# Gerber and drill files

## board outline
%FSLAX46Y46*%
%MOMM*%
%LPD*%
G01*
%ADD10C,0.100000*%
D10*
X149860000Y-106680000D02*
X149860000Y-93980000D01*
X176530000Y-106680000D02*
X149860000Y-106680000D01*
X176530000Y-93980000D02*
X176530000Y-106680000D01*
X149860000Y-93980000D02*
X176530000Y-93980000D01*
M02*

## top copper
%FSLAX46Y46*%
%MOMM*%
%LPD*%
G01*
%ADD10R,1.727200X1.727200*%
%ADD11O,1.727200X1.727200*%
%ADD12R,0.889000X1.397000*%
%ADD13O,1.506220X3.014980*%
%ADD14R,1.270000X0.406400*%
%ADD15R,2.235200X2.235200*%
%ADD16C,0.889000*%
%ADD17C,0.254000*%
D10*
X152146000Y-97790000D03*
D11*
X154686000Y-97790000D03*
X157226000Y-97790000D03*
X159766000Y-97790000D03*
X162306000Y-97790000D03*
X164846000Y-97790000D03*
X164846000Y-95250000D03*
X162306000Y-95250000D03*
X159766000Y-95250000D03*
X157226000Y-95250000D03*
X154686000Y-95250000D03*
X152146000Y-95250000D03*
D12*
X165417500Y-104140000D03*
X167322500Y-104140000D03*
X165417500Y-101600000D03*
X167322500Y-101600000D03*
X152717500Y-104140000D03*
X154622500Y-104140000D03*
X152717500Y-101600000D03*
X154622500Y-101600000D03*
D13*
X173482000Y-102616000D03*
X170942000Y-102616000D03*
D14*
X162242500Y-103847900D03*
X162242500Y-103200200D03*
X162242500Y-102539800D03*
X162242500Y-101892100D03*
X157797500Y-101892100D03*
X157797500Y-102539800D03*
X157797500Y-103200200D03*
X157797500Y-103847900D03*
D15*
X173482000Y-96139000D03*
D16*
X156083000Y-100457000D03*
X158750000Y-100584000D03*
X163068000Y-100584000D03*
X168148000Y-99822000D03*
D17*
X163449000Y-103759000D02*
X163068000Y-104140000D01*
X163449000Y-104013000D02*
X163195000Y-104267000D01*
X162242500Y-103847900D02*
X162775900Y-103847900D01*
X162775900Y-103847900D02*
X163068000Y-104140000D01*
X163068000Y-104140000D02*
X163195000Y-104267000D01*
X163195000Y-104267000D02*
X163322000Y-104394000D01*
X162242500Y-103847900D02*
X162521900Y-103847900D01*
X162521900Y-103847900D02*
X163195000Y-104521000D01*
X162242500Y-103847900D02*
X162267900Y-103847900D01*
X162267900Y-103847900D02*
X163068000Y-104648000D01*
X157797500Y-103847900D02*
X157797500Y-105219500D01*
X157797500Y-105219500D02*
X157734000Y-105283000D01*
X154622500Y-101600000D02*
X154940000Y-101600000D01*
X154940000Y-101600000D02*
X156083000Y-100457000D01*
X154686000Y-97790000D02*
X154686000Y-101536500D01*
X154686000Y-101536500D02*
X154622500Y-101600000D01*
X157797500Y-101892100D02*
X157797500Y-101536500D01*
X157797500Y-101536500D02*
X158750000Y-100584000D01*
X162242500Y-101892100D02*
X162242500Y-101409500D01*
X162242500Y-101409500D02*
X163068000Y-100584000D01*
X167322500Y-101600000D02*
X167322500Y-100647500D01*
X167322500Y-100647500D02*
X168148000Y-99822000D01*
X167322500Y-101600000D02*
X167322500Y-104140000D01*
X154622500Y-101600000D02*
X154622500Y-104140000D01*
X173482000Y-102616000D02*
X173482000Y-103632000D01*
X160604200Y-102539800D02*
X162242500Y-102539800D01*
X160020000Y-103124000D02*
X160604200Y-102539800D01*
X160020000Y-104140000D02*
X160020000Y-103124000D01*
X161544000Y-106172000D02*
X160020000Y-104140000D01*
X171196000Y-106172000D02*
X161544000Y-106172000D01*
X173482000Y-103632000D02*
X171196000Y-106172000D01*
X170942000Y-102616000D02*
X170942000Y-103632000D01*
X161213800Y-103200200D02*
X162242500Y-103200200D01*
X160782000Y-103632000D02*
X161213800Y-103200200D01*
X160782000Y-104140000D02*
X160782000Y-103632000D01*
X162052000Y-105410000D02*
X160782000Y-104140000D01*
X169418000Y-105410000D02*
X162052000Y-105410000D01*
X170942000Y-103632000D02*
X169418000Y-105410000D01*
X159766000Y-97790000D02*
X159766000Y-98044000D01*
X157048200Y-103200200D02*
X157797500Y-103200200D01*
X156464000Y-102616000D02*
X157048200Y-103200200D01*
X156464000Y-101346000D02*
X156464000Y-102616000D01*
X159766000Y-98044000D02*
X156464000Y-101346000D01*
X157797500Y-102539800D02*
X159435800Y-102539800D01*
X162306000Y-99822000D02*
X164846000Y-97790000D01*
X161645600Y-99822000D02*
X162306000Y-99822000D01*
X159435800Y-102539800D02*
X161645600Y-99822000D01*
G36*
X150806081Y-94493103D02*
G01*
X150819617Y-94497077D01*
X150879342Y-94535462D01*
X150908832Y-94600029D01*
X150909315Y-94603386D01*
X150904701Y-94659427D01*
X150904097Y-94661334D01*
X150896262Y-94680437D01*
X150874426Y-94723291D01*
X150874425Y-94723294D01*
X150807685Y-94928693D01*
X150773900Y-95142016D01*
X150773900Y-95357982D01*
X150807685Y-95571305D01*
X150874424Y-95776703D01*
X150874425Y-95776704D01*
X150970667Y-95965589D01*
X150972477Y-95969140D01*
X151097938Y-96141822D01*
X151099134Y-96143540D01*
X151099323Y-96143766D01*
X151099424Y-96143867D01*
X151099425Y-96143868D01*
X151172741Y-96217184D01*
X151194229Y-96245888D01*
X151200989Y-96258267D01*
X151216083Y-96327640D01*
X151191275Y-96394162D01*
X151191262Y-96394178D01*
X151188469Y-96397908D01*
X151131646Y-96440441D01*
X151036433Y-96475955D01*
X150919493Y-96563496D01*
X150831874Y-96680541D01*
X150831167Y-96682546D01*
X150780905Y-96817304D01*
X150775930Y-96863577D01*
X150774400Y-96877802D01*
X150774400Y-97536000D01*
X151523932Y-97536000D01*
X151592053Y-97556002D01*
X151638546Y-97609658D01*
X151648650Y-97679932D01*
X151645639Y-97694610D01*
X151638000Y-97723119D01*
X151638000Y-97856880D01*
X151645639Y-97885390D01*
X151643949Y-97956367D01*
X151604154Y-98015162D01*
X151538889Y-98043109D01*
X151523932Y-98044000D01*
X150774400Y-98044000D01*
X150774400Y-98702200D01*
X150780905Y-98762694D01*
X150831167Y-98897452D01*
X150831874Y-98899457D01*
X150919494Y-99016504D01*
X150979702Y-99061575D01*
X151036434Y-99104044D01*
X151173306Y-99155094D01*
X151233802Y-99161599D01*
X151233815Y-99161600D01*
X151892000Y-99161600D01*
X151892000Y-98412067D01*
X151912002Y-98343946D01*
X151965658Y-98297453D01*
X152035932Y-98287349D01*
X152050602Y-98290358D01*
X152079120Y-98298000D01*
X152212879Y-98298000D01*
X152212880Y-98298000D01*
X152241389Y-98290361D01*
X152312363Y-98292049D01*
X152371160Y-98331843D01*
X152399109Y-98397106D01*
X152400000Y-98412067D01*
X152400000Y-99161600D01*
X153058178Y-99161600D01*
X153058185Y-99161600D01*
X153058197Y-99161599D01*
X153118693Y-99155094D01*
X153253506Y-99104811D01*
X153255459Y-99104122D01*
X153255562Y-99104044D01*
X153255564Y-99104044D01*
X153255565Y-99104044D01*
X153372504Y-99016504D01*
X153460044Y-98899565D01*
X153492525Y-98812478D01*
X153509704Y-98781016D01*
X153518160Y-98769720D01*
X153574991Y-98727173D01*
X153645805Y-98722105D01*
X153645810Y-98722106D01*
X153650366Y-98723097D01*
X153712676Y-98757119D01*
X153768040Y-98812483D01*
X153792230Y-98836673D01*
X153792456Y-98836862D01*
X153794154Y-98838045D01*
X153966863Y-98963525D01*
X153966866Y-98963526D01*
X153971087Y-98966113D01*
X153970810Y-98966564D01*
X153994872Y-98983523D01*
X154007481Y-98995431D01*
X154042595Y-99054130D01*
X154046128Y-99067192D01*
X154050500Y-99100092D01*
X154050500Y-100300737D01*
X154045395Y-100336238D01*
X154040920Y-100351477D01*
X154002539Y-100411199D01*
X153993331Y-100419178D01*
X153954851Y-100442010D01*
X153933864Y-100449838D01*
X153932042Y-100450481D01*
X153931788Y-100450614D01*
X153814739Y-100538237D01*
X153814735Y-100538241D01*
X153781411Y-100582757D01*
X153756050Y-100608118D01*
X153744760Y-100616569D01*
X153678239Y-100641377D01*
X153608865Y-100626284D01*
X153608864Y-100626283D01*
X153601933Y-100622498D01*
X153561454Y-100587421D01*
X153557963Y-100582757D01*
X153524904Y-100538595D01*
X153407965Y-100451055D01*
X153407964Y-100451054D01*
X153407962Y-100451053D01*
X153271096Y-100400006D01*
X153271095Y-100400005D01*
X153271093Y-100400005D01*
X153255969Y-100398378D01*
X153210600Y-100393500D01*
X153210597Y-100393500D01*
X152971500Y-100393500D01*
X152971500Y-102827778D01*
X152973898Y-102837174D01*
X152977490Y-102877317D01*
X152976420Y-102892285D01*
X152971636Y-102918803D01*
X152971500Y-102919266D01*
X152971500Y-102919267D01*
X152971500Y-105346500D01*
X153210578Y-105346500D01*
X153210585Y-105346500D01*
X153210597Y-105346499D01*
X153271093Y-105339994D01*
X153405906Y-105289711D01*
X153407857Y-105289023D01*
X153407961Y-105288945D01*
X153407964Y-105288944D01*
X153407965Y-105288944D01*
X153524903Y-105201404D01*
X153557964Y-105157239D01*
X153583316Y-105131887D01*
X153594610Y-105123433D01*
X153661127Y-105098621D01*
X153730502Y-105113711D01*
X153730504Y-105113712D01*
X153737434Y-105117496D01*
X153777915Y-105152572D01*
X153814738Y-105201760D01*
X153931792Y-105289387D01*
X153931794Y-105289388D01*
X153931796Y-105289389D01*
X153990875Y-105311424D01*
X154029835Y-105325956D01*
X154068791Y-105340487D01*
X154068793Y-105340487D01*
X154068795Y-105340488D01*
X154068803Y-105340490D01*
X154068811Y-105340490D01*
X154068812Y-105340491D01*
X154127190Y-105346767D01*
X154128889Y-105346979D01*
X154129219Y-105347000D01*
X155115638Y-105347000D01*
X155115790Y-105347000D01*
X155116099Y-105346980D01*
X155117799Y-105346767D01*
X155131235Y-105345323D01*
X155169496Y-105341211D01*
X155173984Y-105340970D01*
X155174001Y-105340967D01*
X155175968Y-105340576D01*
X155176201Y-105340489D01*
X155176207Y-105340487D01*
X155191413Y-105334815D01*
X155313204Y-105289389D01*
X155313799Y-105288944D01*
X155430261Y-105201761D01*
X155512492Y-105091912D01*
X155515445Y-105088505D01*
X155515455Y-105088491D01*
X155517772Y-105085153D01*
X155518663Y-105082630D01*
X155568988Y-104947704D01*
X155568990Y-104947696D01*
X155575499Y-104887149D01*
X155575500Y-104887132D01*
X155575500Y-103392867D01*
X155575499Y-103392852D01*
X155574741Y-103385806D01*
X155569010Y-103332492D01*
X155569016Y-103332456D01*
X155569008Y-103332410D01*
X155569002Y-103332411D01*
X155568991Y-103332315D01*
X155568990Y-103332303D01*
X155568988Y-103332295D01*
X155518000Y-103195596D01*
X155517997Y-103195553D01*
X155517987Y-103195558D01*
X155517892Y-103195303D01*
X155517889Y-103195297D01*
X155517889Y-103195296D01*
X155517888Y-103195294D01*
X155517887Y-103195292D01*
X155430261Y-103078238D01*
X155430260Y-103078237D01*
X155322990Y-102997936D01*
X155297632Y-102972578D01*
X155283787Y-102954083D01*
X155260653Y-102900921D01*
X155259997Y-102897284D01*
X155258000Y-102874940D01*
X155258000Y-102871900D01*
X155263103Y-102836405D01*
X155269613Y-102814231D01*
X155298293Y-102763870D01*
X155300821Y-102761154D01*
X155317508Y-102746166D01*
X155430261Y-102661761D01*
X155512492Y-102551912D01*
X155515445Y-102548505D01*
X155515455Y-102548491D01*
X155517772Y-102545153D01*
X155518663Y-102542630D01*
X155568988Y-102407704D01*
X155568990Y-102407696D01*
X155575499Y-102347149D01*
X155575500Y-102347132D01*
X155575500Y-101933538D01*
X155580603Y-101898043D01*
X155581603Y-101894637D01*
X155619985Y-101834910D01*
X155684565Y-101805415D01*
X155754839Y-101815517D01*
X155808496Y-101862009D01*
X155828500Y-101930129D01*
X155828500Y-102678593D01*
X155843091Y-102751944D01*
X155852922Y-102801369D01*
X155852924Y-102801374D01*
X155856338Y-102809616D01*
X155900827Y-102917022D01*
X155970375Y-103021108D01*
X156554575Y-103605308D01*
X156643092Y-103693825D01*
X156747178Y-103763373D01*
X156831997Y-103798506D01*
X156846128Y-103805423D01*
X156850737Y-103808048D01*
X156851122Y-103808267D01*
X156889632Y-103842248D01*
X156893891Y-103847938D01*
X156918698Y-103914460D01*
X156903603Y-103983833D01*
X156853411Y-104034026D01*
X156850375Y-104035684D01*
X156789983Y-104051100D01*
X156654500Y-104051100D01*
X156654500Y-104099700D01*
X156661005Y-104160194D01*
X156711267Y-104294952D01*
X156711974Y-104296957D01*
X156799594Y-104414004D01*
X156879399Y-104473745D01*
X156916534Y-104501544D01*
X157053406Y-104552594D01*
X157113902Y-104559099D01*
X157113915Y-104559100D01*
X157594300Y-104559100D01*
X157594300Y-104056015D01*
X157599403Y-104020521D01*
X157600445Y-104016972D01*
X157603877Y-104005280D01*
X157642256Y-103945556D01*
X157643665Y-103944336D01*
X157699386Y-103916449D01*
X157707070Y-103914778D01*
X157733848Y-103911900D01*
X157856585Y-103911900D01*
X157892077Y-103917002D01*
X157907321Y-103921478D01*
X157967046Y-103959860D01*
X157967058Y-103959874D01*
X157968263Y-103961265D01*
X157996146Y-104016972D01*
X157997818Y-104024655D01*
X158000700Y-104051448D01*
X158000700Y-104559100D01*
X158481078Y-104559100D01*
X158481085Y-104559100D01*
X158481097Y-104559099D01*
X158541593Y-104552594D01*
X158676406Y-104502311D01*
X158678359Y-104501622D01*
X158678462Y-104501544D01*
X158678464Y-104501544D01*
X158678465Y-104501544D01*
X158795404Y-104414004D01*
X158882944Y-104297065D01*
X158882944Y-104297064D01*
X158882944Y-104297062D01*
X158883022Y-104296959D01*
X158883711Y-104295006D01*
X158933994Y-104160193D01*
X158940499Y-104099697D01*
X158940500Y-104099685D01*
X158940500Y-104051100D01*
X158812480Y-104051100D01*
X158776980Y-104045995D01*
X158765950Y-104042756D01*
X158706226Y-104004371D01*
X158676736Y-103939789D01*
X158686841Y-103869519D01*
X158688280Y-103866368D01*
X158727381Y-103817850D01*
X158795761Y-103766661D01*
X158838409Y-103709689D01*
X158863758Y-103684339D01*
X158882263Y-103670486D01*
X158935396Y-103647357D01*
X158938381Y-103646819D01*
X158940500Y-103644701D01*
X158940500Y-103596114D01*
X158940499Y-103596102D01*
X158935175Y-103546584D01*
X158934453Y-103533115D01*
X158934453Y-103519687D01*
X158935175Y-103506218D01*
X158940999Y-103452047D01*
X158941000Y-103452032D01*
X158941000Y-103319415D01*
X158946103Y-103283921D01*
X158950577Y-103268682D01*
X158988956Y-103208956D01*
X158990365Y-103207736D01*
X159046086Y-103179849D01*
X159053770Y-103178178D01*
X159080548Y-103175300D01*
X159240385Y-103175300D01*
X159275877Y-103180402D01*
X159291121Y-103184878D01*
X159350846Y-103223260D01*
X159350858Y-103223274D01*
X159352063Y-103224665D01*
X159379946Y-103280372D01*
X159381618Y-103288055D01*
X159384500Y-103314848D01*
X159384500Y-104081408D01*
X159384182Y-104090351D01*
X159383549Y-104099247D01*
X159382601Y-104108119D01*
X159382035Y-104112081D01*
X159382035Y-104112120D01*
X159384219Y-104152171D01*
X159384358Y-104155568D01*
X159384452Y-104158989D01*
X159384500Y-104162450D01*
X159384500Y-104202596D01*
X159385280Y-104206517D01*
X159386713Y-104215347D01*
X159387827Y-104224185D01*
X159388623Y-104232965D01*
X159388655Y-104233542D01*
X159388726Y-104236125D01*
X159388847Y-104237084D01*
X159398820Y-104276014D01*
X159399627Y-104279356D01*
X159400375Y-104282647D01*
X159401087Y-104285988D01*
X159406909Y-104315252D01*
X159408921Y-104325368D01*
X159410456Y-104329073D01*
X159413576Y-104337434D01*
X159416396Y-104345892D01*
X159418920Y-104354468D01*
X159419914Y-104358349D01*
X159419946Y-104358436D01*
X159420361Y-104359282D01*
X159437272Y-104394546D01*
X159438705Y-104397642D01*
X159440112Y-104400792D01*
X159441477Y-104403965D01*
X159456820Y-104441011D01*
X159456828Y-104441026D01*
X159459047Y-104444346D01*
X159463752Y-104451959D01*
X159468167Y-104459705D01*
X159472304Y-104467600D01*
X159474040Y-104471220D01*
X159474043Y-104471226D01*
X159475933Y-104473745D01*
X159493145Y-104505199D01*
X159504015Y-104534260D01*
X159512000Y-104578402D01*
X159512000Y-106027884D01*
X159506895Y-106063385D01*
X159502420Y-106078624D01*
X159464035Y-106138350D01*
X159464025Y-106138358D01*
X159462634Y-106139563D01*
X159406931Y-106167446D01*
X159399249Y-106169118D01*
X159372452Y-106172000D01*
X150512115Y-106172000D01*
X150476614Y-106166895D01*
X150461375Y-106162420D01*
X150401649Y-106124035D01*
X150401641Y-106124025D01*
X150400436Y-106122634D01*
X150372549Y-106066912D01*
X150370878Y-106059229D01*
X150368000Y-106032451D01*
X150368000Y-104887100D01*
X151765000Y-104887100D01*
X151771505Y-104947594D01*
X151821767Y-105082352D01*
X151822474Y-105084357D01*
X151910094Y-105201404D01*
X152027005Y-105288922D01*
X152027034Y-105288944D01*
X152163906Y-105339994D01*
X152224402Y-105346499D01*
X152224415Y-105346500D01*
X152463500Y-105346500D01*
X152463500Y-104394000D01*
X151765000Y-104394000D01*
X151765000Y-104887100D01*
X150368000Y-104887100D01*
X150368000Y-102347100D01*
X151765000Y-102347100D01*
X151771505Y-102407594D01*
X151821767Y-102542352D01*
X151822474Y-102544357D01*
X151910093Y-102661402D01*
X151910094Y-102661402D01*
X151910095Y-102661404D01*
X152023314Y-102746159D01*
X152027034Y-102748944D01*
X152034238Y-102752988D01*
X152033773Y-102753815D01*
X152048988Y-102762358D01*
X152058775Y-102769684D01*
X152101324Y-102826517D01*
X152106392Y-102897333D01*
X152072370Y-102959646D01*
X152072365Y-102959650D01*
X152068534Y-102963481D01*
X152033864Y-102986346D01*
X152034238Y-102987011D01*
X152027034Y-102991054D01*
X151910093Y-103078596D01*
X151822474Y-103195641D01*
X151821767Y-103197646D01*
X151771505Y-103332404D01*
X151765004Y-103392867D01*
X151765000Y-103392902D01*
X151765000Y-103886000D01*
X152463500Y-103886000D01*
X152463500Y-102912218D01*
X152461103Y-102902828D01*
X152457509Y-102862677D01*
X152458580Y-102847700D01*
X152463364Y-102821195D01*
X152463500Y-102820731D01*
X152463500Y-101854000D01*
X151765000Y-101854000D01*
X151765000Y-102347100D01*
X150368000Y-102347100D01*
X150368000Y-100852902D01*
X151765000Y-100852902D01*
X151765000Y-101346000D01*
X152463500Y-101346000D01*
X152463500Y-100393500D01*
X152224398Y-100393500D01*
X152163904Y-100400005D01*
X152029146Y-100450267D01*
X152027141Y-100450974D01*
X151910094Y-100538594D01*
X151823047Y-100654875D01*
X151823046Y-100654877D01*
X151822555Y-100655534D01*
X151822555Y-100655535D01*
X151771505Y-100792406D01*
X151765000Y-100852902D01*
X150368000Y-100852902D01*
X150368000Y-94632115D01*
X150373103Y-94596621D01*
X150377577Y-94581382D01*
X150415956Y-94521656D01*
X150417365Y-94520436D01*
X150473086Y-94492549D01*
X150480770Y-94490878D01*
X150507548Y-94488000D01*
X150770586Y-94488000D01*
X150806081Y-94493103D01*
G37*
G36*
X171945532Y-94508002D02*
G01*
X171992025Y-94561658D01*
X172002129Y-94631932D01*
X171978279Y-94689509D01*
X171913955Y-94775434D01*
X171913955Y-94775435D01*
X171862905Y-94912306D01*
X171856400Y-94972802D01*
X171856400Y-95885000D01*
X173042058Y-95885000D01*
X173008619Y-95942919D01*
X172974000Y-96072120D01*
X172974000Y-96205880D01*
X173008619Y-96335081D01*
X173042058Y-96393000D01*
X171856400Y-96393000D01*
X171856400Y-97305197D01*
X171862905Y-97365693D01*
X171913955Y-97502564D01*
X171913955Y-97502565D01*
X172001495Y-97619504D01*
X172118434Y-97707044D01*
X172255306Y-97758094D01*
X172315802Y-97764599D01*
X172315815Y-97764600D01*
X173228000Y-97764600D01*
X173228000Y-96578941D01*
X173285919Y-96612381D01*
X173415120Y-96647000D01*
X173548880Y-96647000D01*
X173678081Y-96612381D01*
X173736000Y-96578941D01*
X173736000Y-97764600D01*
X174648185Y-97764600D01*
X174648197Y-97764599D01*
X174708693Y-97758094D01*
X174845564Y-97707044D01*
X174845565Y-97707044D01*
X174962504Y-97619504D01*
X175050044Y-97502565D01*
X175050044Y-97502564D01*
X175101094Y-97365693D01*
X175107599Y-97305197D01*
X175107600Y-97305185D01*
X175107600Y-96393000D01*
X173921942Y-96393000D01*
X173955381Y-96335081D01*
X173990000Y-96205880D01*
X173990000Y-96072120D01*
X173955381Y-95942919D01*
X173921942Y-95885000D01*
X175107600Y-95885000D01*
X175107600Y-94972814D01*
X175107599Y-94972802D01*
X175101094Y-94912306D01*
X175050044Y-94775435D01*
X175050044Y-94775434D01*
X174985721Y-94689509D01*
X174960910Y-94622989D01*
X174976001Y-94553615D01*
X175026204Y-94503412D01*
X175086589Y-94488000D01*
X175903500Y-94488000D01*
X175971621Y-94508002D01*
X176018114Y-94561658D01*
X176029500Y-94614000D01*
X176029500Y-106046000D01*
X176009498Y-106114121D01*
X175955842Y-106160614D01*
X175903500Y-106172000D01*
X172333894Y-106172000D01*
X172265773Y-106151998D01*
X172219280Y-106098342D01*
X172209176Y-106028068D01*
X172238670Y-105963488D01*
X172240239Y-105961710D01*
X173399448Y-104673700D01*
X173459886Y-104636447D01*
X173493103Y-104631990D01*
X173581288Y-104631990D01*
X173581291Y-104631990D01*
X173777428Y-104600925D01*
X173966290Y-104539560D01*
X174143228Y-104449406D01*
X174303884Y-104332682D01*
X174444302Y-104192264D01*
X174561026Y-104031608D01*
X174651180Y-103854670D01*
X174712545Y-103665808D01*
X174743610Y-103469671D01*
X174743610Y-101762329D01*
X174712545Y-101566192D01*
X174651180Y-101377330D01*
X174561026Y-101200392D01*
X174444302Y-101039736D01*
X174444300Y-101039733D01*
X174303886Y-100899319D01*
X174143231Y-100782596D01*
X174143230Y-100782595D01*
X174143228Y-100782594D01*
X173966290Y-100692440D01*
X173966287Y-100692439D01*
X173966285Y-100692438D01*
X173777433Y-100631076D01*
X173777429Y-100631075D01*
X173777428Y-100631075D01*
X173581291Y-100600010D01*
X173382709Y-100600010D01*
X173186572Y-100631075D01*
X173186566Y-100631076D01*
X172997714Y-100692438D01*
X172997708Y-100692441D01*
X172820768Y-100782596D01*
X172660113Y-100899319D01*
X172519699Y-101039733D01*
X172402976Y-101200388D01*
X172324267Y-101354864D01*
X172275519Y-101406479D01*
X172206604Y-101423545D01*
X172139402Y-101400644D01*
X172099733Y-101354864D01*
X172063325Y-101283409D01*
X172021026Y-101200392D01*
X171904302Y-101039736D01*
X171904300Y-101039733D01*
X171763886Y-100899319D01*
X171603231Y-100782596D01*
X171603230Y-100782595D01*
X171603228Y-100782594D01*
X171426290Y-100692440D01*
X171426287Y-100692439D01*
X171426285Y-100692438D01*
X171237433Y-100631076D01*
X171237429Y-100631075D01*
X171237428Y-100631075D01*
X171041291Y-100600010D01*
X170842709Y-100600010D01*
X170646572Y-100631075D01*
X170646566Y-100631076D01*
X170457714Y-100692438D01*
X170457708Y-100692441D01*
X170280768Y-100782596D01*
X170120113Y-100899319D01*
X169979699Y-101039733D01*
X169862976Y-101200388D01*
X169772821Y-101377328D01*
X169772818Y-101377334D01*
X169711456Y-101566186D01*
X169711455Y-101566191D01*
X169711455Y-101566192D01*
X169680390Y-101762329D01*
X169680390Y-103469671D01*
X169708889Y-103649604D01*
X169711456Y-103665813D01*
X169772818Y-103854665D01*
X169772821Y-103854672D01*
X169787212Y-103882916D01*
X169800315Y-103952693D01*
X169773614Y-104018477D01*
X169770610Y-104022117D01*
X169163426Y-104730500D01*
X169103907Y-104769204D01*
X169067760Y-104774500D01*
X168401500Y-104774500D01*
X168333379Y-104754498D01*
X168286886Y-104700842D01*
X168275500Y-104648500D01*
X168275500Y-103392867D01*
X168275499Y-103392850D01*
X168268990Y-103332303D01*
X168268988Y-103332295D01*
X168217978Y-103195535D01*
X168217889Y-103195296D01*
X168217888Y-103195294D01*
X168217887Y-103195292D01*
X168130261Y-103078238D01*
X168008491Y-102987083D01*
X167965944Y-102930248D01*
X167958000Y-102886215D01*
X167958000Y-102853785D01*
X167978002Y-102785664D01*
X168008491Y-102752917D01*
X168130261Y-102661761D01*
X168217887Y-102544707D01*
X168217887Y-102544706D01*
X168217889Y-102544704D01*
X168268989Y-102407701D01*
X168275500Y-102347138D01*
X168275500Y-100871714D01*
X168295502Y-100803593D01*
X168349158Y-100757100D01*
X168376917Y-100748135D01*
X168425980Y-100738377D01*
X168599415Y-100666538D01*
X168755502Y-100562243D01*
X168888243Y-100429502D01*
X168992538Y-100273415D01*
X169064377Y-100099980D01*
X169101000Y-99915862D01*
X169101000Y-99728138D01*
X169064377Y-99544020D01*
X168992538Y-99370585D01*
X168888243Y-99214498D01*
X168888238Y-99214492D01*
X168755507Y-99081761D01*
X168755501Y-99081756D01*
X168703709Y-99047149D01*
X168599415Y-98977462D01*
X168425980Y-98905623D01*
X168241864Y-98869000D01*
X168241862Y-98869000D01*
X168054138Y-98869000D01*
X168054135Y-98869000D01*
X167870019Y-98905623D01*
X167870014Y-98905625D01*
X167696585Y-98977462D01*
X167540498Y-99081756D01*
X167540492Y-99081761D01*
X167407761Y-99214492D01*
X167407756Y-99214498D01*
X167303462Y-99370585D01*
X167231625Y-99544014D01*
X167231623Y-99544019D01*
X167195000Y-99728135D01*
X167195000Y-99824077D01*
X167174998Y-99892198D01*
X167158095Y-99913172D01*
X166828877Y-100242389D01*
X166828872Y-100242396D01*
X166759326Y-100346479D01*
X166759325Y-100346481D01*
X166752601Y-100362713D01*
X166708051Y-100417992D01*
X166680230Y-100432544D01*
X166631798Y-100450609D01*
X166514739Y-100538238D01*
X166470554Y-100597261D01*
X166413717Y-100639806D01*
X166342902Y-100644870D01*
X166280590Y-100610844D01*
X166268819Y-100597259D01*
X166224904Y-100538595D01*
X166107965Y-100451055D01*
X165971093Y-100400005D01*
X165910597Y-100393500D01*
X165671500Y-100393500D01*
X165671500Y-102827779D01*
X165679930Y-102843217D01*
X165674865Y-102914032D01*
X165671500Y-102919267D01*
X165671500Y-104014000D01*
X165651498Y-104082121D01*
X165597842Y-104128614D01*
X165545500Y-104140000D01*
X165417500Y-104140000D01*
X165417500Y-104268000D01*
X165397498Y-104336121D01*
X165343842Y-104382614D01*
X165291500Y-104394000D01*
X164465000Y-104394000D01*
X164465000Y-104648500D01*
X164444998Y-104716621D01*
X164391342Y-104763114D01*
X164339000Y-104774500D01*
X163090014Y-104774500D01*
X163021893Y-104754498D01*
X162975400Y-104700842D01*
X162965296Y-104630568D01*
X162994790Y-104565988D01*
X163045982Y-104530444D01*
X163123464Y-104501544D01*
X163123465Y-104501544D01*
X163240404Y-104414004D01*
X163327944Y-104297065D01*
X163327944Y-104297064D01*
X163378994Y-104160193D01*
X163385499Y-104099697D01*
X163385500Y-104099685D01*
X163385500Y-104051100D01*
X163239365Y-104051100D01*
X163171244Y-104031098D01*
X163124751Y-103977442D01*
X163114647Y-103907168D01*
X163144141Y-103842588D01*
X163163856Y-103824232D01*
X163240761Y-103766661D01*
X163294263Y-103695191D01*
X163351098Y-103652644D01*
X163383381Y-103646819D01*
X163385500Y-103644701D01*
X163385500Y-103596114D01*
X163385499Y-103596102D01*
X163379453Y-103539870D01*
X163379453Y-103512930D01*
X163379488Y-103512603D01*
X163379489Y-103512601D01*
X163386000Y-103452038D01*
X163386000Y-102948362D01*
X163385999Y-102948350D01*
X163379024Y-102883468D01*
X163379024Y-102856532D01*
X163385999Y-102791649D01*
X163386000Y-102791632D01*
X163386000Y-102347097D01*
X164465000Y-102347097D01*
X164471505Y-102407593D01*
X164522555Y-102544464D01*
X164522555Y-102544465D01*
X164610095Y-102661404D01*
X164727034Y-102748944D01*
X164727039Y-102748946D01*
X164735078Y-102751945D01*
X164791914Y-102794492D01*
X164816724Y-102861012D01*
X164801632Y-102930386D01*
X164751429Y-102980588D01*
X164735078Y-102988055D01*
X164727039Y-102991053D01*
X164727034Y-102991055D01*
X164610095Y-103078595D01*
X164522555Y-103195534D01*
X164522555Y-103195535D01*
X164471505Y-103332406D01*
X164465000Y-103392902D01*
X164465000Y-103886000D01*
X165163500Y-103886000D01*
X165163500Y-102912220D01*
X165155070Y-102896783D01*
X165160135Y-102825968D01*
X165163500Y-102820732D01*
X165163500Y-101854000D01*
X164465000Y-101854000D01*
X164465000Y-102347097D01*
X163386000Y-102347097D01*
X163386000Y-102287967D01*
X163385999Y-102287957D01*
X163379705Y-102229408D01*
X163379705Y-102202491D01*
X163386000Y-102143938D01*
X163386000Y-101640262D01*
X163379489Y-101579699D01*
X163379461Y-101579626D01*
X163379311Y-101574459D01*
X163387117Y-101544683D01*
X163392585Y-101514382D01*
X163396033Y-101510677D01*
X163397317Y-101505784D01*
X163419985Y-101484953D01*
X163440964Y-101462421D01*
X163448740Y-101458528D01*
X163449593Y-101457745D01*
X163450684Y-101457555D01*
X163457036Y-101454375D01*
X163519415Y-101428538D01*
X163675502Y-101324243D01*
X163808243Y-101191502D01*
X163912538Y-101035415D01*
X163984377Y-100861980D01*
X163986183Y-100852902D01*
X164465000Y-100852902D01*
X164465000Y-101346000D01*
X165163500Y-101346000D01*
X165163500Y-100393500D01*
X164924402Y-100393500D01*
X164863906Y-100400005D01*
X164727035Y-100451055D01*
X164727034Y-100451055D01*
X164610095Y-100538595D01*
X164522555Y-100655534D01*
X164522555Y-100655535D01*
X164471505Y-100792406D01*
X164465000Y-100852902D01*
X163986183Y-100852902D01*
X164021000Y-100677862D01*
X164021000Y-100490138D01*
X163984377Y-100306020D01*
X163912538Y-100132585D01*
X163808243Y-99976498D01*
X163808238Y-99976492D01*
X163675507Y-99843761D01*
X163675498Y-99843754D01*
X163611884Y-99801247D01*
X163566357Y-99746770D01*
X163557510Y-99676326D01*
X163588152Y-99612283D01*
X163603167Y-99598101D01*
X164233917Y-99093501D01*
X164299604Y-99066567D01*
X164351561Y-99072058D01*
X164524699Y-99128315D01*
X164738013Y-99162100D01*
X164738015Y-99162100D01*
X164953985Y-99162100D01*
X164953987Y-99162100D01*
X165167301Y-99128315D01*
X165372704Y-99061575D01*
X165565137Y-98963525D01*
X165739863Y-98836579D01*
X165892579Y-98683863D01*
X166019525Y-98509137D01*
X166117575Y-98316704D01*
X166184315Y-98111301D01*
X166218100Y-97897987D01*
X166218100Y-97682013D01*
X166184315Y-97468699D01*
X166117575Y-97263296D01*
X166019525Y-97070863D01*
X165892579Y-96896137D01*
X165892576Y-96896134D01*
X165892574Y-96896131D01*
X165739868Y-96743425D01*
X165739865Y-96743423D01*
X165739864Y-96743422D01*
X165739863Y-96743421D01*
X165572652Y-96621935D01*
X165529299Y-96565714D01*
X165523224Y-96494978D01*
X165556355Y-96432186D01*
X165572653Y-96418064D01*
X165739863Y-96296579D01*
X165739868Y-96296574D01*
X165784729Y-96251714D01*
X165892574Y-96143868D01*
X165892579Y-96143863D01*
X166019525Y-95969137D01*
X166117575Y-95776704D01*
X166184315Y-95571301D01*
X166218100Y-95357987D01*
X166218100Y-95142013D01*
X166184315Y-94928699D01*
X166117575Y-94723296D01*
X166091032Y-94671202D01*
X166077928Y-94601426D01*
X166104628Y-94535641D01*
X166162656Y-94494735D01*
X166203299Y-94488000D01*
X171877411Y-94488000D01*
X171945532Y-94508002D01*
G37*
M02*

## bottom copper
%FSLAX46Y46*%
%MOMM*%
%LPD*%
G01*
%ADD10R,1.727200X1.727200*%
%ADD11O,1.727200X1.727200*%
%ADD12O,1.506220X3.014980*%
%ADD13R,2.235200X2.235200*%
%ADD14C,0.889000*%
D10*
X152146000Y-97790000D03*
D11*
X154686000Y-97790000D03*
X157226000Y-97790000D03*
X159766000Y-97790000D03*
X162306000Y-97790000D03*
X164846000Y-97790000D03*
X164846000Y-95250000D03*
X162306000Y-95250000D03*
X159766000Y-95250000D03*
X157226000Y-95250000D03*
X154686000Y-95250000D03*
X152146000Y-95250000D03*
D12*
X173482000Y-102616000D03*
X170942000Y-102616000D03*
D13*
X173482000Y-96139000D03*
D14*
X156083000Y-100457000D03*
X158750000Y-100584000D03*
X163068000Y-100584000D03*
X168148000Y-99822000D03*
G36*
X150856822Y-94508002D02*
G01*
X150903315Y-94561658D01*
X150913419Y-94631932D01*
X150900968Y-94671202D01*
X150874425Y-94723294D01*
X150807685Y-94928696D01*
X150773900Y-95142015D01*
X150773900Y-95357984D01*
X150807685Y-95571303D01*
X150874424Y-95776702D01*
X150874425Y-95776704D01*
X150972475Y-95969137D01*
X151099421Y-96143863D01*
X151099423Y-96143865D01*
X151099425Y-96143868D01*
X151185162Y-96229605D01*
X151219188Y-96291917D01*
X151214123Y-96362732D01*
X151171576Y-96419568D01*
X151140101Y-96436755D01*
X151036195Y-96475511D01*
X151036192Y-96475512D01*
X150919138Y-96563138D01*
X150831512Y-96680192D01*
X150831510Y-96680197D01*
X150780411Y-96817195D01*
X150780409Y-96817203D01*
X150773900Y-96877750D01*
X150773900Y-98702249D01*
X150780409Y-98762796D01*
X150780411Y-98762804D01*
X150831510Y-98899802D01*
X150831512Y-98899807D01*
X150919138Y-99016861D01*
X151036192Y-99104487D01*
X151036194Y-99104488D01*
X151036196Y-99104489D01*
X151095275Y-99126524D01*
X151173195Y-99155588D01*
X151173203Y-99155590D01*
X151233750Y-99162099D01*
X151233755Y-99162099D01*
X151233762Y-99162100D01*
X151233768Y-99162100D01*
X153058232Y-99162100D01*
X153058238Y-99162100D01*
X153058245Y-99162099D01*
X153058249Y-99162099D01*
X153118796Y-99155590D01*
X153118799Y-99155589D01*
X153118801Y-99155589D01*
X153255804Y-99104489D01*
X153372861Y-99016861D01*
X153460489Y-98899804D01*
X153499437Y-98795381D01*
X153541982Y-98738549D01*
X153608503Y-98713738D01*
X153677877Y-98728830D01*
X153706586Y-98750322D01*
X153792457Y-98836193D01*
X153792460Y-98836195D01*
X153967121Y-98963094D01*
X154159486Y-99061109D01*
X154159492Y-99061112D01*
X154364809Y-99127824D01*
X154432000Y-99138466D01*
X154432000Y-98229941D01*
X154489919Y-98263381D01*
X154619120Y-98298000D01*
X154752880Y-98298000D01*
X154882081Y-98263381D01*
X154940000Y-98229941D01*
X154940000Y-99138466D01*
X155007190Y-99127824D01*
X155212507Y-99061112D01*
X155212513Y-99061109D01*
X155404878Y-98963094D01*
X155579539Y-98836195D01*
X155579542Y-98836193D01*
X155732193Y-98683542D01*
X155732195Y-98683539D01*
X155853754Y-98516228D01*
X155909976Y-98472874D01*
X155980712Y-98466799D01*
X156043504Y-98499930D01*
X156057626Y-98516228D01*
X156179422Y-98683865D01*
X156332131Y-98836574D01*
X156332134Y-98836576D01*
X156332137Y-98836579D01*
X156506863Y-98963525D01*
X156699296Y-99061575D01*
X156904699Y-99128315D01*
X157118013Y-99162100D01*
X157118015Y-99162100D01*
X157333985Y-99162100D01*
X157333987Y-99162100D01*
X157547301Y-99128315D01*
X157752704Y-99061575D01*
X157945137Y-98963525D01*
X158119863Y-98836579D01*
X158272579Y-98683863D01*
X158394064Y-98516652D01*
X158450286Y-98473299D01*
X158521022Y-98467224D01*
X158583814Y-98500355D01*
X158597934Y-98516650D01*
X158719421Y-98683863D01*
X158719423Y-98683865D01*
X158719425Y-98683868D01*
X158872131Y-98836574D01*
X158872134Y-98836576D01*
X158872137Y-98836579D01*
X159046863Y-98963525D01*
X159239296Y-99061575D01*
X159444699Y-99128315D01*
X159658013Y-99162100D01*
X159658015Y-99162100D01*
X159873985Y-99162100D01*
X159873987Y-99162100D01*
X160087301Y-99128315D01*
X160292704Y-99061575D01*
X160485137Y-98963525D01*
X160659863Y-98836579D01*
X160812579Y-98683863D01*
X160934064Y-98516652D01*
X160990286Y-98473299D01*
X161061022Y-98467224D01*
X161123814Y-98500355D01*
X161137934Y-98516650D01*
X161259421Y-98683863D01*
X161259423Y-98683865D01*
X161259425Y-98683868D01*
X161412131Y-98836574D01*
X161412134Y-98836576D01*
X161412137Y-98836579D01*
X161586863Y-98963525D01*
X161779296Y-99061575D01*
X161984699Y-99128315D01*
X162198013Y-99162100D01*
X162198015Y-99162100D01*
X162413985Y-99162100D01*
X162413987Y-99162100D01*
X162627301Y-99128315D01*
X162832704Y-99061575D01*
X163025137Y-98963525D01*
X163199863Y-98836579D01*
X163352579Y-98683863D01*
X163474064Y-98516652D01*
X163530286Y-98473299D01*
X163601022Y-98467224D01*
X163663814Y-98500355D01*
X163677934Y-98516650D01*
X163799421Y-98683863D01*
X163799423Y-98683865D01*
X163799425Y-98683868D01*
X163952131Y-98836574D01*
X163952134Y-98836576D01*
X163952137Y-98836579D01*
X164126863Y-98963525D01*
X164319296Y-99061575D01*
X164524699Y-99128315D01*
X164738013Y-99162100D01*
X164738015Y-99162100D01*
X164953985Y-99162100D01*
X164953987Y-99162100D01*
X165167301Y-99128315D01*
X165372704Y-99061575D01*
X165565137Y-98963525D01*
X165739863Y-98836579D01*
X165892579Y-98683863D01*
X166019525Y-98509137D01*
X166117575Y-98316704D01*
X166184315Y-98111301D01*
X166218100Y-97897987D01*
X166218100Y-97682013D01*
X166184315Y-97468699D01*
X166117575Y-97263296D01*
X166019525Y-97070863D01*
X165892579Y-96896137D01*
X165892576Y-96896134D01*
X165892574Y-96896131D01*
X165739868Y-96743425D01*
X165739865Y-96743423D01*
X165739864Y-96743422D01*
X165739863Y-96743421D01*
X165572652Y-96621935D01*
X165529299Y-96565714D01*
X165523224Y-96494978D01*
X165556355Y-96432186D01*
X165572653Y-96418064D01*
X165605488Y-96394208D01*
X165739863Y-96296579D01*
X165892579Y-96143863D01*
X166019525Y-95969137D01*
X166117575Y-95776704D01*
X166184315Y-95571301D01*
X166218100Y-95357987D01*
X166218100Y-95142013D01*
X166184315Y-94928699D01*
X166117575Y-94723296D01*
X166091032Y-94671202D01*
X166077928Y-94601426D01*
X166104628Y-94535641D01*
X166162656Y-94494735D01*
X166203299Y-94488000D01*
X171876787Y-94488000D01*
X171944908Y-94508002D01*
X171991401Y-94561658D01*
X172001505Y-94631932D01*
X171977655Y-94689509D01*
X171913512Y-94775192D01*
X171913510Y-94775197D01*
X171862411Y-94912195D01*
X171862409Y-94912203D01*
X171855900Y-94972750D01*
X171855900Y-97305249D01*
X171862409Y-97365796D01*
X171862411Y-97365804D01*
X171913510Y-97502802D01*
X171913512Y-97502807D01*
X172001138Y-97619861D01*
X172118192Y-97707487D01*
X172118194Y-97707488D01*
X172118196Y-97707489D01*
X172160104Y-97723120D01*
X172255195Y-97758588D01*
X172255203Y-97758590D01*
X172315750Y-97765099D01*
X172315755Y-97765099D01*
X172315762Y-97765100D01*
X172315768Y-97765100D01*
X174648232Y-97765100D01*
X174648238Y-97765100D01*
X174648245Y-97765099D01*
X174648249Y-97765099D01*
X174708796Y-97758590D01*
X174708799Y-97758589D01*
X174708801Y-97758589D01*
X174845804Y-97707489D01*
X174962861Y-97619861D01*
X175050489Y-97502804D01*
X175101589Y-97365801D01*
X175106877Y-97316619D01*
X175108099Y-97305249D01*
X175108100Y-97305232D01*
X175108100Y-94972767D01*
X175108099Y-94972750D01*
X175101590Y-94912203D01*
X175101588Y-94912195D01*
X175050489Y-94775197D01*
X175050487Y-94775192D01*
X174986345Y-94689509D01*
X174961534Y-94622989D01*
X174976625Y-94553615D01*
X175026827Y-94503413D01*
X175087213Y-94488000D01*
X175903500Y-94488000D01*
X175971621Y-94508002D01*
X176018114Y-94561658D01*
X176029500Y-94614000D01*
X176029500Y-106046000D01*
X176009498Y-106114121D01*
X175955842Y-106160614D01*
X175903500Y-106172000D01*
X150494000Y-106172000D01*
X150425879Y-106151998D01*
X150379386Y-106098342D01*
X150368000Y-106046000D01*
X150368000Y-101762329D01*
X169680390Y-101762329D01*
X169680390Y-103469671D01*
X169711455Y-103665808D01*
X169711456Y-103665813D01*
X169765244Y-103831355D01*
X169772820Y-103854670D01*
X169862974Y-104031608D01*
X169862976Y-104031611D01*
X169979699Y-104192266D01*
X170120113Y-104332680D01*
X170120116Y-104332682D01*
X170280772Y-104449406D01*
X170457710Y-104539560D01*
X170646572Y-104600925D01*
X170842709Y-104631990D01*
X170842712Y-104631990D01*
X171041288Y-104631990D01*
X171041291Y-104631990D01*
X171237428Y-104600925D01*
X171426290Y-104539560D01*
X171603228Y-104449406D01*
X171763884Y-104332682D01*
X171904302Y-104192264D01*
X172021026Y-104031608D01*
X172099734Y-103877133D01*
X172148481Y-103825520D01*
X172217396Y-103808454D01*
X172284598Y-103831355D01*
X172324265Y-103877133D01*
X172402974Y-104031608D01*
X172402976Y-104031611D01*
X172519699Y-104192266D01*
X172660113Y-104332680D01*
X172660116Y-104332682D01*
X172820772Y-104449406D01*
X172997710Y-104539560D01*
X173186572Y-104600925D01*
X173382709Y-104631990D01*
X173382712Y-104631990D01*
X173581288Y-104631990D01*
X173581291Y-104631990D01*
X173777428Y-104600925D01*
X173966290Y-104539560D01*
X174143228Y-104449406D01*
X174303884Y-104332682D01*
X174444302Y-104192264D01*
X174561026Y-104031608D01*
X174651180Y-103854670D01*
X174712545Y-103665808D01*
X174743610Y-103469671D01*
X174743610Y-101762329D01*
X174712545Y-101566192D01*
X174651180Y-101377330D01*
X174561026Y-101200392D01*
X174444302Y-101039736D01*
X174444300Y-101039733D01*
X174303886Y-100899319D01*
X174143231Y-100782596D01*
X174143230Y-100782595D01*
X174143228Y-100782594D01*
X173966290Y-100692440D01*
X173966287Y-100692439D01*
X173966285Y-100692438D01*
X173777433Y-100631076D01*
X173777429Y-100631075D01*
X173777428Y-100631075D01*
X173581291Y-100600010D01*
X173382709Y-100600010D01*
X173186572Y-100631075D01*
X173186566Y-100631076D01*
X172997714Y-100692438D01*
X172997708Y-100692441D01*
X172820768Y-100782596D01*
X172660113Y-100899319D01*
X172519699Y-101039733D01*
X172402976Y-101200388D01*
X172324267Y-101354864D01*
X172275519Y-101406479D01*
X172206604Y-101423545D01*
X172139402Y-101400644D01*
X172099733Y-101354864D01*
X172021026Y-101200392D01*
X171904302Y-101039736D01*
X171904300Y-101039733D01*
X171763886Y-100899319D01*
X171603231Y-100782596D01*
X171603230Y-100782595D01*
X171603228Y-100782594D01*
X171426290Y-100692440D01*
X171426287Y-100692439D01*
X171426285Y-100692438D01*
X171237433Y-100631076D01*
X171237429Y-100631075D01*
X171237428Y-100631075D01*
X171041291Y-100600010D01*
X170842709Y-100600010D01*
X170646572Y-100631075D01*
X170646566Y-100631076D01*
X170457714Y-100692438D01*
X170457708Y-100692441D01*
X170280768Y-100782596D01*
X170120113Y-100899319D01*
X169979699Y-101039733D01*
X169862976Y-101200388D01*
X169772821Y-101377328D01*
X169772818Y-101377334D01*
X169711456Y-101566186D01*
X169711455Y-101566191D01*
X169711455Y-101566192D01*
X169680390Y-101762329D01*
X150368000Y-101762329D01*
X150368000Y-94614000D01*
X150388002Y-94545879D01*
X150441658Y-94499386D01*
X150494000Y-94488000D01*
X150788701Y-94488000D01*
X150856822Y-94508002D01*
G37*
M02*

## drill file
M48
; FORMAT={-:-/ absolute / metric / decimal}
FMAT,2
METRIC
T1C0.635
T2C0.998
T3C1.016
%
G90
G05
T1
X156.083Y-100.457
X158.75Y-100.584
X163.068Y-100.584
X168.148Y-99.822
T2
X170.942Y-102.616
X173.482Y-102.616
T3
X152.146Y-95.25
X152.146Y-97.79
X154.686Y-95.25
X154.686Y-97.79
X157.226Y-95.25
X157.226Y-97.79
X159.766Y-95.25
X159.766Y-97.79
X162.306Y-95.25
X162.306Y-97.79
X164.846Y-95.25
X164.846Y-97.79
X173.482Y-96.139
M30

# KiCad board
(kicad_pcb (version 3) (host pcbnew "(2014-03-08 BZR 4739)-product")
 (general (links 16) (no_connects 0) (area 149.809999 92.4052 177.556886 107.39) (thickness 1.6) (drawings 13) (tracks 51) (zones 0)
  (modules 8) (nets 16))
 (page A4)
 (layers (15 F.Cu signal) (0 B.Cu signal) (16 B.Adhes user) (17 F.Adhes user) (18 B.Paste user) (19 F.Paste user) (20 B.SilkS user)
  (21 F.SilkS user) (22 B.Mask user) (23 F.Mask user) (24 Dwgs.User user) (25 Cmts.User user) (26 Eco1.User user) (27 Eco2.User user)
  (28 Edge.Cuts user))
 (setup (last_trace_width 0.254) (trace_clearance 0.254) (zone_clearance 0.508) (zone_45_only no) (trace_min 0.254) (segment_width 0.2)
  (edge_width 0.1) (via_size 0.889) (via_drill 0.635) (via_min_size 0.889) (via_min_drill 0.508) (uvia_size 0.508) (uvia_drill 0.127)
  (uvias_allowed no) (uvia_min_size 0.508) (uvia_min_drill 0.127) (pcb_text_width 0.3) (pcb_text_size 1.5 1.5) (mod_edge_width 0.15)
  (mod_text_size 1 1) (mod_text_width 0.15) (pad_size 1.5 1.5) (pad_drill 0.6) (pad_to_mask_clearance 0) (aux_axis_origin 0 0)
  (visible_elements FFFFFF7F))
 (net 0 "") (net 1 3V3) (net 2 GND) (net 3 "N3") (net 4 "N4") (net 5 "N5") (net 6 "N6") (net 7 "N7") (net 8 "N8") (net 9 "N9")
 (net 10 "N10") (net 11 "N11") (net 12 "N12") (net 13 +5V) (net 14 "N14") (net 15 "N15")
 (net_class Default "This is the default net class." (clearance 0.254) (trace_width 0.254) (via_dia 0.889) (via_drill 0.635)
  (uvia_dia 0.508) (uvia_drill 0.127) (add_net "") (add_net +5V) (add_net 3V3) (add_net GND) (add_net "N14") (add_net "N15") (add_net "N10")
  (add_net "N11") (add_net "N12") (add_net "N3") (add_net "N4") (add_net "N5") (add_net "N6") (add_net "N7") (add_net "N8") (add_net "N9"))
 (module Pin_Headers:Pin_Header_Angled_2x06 (layer F.Cu) (at 158.496 96.52)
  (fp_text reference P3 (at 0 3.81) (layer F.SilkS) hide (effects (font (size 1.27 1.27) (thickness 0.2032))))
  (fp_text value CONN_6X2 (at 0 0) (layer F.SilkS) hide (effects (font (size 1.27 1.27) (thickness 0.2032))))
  (pad 1 thru_hole rect (at -6.35 1.27) (size 1.7272 1.7272) (drill 1.016) (layers *.Cu *.Mask F.SilkS) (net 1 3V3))
  (pad 2 thru_hole oval (at -3.81 1.27) (size 1.7272 1.7272) (drill 1.016) (layers *.Cu *.Mask F.SilkS) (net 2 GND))
  (pad 3 thru_hole oval (at -1.27 1.27) (size 1.7272 1.7272) (drill 1.016) (layers *.Cu *.Mask F.SilkS) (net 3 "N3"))
  (pad 4 thru_hole oval (at 1.27 1.27) (size 1.7272 1.7272) (drill 1.016) (layers *.Cu *.Mask F.SilkS) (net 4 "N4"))
  (pad 5 thru_hole oval (at 3.81 1.27) (size 1.7272 1.7272) (drill 1.016) (layers *.Cu *.Mask F.SilkS) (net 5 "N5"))
  (pad 6 thru_hole oval (at 6.35 1.27) (size 1.7272 1.7272) (drill 1.016) (layers *.Cu *.Mask F.SilkS) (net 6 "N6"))
  (pad 7 thru_hole oval (at 6.35 -1.27) (size 1.7272 1.7272) (drill 1.016) (layers *.Cu *.Mask F.SilkS) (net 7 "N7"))
  (pad 8 thru_hole oval (at 3.81 -1.27) (size 1.7272 1.7272) (drill 1.016) (layers *.Cu *.Mask F.SilkS) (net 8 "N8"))
  (pad 9 thru_hole oval (at 1.27 -1.27) (size 1.7272 1.7272) (drill 1.016) (layers *.Cu *.Mask F.SilkS) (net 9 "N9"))
  (pad 10 thru_hole oval (at -1.27 -1.27) (size 1.7272 1.7272) (drill 1.016) (layers *.Cu *.Mask F.SilkS) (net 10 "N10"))
  (pad 11 thru_hole oval (at -3.81 -1.27) (size 1.7272 1.7272) (drill 1.016) (layers *.Cu *.Mask F.SilkS) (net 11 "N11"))
  (pad 12 thru_hole oval (at -6.35 -1.27) (size 1.7272 1.7272) (drill 1.016) (layers *.Cu *.Mask F.SilkS) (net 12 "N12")))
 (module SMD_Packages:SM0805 (layer F.Cu) (at 166.37 104.14)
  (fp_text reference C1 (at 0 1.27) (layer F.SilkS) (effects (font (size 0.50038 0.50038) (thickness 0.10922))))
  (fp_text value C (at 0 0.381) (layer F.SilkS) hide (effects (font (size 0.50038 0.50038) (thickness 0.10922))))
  (pad 1 smd rect (at -0.9525 0) (size 0.889 1.397) (layers F.Cu F.Paste F.Mask) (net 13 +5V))
  (pad 2 smd rect (at 0.9525 0) (size 0.889 1.397) (layers F.Cu F.Paste F.Mask) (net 2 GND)))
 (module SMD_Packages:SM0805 (layer F.Cu) (at 166.37 101.6)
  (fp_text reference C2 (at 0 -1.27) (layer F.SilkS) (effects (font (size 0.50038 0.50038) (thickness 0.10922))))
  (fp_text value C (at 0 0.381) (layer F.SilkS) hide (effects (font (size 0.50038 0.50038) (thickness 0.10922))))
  (pad 1 smd rect (at -0.9525 0) (size 0.889 1.397) (layers F.Cu F.Paste F.Mask) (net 13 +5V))
  (pad 2 smd rect (at 0.9525 0) (size 0.889 1.397) (layers F.Cu F.Paste F.Mask) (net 2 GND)))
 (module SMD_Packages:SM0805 (layer F.Cu) (at 153.67 104.14)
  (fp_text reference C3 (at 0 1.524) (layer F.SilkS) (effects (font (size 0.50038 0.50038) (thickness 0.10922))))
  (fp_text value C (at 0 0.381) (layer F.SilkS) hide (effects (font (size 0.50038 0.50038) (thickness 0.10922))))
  (pad 1 smd rect (at -0.9525 0) (size 0.889 1.397) (layers F.Cu F.Paste F.Mask) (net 1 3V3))
  (pad 2 smd rect (at 0.9525 0) (size 0.889 1.397) (layers F.Cu F.Paste F.Mask) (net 2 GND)))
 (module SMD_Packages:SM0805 (layer F.Cu) (at 153.67 101.6)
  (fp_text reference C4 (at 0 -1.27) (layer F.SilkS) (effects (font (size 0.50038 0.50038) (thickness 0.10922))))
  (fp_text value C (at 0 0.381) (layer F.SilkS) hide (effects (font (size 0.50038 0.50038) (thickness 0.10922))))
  (pad 1 smd rect (at -0.9525 0) (size 0.889 1.397) (layers F.Cu F.Paste F.Mask) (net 1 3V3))
  (pad 2 smd rect (at 0.9525 0) (size 0.889 1.397) (layers F.Cu F.Paste F.Mask) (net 2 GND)))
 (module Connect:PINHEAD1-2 (layer F.Cu) (at 172.212 102.616 180)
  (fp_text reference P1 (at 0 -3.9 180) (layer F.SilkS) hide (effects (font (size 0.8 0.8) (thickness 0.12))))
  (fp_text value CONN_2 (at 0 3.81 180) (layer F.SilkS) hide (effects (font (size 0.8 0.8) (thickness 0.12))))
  (pad 1 thru_hole oval (at -1.27 0 180) (size 1.50622 3.01498) (drill 0.99822) (layers *.Cu *.Mask F.SilkS) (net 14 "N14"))
  (pad 2 thru_hole oval (at 1.27 0 180) (size 1.50622 3.01498) (drill 0.99822) (layers *.Cu *.Mask F.SilkS) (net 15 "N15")))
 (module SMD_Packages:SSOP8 (layer F.Cu) (at 160.02 102.87 90)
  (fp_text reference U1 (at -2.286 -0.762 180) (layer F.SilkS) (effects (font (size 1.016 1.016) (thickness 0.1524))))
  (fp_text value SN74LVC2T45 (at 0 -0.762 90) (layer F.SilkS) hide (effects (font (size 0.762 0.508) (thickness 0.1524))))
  (pad 1 smd rect (at -0.9779 2.2225 90) (size 0.4064 1.27) (layers F.Cu F.Paste F.Mask) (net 13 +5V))
  (pad 2 smd rect (at -0.3302 2.2225 90) (size 0.4064 1.27) (layers F.Cu F.Paste F.Mask) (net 15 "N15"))
  (pad 3 smd rect (at 0.3302 2.2225 90) (size 0.4064 1.27) (layers F.Cu F.Paste F.Mask) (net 14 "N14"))
  (pad 4 smd rect (at 0.9779 2.2225 90) (size 0.4064 1.27) (layers F.Cu F.Paste F.Mask) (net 2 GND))
  (pad 5 smd rect (at 0.9779 -2.2225 90) (size 0.4064 1.27) (layers F.Cu F.Paste F.Mask) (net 2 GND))
  (pad 6 smd rect (at 0.3302 -2.2225 90) (size 0.4064 1.27) (layers F.Cu F.Paste F.Mask) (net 6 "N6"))
  (pad 7 smd rect (at -0.3302 -2.2225 90) (size 0.4064 1.27) (layers F.Cu F.Paste F.Mask) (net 4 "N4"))
  (pad 8 smd rect (at -0.9779 -2.2225 90) (size 0.4064 1.27) (layers F.Cu F.Paste F.Mask) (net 1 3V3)))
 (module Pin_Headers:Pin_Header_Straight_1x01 (layer F.Cu) (at 173.482 96.139)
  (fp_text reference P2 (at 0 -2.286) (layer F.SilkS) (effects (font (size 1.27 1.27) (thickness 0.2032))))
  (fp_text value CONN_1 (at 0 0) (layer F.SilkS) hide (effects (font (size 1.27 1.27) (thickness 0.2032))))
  (pad 1 thru_hole rect (at 0 0) (size 2.2352 2.2352) (drill 1.016) (layers *.Cu *.Mask F.SilkS) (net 13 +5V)))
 (gr_line (start 149.86 106.68) (end 149.86 93.98) (angle 90) (layer Edge.Cuts) (width 0.1))
 (gr_line (start 176.53 106.68) (end 149.86 106.68) (angle 90) (layer Edge.Cuts) (width 0.1))
 (gr_line (start 176.53 93.98) (end 176.53 106.68) (angle 90) (layer Edge.Cuts) (width 0.1))
 (gr_line (start 149.86 93.98) (end 176.53 93.98) (angle 90) (layer Edge.Cuts) (width 0.1))
 (segment (start 163.449 103.759) (end 163.068 104.14) (width 0.254) (layer F.Cu) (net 13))
 (segment (start 163.449 104.013) (end 163.195 104.267) (width 0.254) (layer F.Cu) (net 13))
 (segment (start 162.2425 103.8479) (end 162.7759 103.8479) (width 0.254) (layer F.Cu) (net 13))
 (segment (start 162.7759 103.8479) (end 163.068 104.14) (width 0.254) (layer F.Cu) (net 13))
 (segment (start 163.068 104.14) (end 163.195 104.267) (width 0.254) (layer F.Cu) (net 13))
 (segment (start 163.195 104.267) (end 163.322 104.394) (width 0.254) (layer F.Cu) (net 13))
 (segment (start 162.2425 103.8479) (end 162.5219 103.8479) (width 0.254) (layer F.Cu) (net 13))
 (segment (start 162.5219 103.8479) (end 163.195 104.521) (width 0.254) (layer F.Cu) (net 13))
 (segment (start 162.2425 103.8479) (end 162.2679 103.8479) (width 0.254) (layer F.Cu) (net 13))
 (segment (start 162.2679 103.8479) (end 163.068 104.648) (width 0.254) (layer F.Cu) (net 13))
 (segment (start 157.7975 103.8479) (end 157.7975 105.2195) (width 0.254) (layer F.Cu) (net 1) (status 400000))
 (segment (start 157.7975 105.2195) (end 157.734 105.283) (width 0.254) (layer F.Cu) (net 1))
 (segment (start 154.6225 101.6) (end 154.94 101.6) (width 0.254) (layer F.Cu) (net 2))
 (via (at 156.083 100.457) (size 0.889) (layers F.Cu B.Cu) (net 2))
 (segment (start 154.94 101.6) (end 156.083 100.457) (width 0.254) (layer F.Cu) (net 2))
 (segment (start 154.686 97.79) (end 154.686 101.5365) (width 0.254) (layer F.Cu) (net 2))
 (segment (start 154.686 101.5365) (end 154.6225 101.6) (width 0.254) (layer F.Cu) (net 2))
 (segment (start 157.7975 101.8921) (end 157.7975 101.5365) (width 0.254) (layer F.Cu) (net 2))
 (via (at 158.75 100.584) (size 0.889) (layers F.Cu B.Cu) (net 2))
 (segment (start 157.7975 101.5365) (end 158.75 100.584) (width 0.254) (layer F.Cu) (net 2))
 (segment (start 162.2425 101.8921) (end 162.2425 101.4095) (width 0.254) (layer F.Cu) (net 2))
 (via (at 163.068 100.584) (size 0.889) (layers F.Cu B.Cu) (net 2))
 (segment (start 162.2425 101.4095) (end 163.068 100.584) (width 0.254) (layer F.Cu) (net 2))
 (segment (start 167.3225 101.6) (end 167.3225 100.6475) (width 0.254) (layer F.Cu) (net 2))
 (via (at 168.148 99.822) (size 0.889) (layers F.Cu B.Cu) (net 2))
 (segment (start 167.3225 100.6475) (end 168.148 99.822) (width 0.254) (layer F.Cu) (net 2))
 (segment (start 167.3225 101.6) (end 167.3225 104.14) (width 0.254) (layer F.Cu) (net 2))
 (segment (start 154.6225 101.6) (end 154.6225 104.14) (width 0.254) (layer F.Cu) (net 2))
 (segment (start 173.482 102.616) (end 173.482 103.632) (width 0.254) (layer F.Cu) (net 14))
 (segment (start 160.6042 102.5398) (end 162.2425 102.5398) (width 0.254) (layer F.Cu) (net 14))
 (segment (start 160.02 103.124) (end 160.6042 102.5398) (width 0.254) (layer F.Cu) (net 14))
 (segment (start 160.02 104.14) (end 160.02 103.124) (width 0.254) (layer F.Cu) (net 14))
 (segment (start 161.544 106.172) (end 160.02 104.14) (width 0.254) (layer F.Cu) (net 14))
 (segment (start 171.196 106.172) (end 161.544 106.172) (width 0.254) (layer F.Cu) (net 14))
 (segment (start 173.482 103.632) (end 171.196 106.172) (width 0.254) (layer F.Cu) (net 14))
 (segment (start 170.942 102.616) (end 170.942 103.632) (width 0.254) (layer F.Cu) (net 15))
 (segment (start 161.2138 103.2002) (end 162.2425 103.2002) (width 0.254) (layer F.Cu) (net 15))
 (segment (start 160.782 103.632) (end 161.2138 103.2002) (width 0.254) (layer F.Cu) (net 15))
 (segment (start 160.782 104.14) (end 160.782 103.632) (width 0.254) (layer F.Cu) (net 15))
 (segment (start 162.052 105.41) (end 160.782 104.14) (width 0.254) (layer F.Cu) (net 15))
 (segment (start 169.418 105.41) (end 162.052 105.41) (width 0.254) (layer F.Cu) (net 15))
 (segment (start 170.942 103.632) (end 169.418 105.41) (width 0.254) (layer F.Cu) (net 15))
 (segment (start 159.766 97.79) (end 159.766 98.044) (width 0.254) (layer F.Cu) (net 4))
 (segment (start 157.0482 103.2002) (end 157.7975 103.2002) (width 0.254) (layer F.Cu) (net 4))
 (segment (start 156.464 102.616) (end 157.0482 103.2002) (width 0.254) (layer F.Cu) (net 4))
 (segment (start 156.464 101.346) (end 156.464 102.616) (width 0.254) (layer F.Cu) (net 4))
 (segment (start 159.766 98.044) (end 156.464 101.346) (width 0.254) (layer F.Cu) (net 4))
 (segment (start 157.7975 102.5398) (end 159.4358 102.5398) (width 0.254) (layer F.Cu) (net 6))
 (segment (start 162.306 99.822) (end 164.846 97.79) (width 0.254) (layer F.Cu) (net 6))
 (segment (start 161.6456 99.822) (end 162.306 99.822) (width 0.254) (layer F.Cu) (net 6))
 (segment (start 159.4358 102.5398) (end 161.6456 99.822) (width 0.254) (layer F.Cu) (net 6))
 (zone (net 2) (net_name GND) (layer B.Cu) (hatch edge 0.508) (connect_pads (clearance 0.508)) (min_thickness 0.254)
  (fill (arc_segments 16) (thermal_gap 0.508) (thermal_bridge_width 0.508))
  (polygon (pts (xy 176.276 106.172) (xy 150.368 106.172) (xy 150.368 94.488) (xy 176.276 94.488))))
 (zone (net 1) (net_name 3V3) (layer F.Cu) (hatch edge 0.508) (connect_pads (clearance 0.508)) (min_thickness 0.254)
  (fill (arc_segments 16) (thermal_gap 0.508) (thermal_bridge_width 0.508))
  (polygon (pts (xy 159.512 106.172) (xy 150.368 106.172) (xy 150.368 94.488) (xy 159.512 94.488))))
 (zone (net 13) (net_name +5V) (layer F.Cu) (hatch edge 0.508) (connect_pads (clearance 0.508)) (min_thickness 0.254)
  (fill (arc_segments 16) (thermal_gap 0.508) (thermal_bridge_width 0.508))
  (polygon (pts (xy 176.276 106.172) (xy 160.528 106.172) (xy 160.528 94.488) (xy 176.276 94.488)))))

